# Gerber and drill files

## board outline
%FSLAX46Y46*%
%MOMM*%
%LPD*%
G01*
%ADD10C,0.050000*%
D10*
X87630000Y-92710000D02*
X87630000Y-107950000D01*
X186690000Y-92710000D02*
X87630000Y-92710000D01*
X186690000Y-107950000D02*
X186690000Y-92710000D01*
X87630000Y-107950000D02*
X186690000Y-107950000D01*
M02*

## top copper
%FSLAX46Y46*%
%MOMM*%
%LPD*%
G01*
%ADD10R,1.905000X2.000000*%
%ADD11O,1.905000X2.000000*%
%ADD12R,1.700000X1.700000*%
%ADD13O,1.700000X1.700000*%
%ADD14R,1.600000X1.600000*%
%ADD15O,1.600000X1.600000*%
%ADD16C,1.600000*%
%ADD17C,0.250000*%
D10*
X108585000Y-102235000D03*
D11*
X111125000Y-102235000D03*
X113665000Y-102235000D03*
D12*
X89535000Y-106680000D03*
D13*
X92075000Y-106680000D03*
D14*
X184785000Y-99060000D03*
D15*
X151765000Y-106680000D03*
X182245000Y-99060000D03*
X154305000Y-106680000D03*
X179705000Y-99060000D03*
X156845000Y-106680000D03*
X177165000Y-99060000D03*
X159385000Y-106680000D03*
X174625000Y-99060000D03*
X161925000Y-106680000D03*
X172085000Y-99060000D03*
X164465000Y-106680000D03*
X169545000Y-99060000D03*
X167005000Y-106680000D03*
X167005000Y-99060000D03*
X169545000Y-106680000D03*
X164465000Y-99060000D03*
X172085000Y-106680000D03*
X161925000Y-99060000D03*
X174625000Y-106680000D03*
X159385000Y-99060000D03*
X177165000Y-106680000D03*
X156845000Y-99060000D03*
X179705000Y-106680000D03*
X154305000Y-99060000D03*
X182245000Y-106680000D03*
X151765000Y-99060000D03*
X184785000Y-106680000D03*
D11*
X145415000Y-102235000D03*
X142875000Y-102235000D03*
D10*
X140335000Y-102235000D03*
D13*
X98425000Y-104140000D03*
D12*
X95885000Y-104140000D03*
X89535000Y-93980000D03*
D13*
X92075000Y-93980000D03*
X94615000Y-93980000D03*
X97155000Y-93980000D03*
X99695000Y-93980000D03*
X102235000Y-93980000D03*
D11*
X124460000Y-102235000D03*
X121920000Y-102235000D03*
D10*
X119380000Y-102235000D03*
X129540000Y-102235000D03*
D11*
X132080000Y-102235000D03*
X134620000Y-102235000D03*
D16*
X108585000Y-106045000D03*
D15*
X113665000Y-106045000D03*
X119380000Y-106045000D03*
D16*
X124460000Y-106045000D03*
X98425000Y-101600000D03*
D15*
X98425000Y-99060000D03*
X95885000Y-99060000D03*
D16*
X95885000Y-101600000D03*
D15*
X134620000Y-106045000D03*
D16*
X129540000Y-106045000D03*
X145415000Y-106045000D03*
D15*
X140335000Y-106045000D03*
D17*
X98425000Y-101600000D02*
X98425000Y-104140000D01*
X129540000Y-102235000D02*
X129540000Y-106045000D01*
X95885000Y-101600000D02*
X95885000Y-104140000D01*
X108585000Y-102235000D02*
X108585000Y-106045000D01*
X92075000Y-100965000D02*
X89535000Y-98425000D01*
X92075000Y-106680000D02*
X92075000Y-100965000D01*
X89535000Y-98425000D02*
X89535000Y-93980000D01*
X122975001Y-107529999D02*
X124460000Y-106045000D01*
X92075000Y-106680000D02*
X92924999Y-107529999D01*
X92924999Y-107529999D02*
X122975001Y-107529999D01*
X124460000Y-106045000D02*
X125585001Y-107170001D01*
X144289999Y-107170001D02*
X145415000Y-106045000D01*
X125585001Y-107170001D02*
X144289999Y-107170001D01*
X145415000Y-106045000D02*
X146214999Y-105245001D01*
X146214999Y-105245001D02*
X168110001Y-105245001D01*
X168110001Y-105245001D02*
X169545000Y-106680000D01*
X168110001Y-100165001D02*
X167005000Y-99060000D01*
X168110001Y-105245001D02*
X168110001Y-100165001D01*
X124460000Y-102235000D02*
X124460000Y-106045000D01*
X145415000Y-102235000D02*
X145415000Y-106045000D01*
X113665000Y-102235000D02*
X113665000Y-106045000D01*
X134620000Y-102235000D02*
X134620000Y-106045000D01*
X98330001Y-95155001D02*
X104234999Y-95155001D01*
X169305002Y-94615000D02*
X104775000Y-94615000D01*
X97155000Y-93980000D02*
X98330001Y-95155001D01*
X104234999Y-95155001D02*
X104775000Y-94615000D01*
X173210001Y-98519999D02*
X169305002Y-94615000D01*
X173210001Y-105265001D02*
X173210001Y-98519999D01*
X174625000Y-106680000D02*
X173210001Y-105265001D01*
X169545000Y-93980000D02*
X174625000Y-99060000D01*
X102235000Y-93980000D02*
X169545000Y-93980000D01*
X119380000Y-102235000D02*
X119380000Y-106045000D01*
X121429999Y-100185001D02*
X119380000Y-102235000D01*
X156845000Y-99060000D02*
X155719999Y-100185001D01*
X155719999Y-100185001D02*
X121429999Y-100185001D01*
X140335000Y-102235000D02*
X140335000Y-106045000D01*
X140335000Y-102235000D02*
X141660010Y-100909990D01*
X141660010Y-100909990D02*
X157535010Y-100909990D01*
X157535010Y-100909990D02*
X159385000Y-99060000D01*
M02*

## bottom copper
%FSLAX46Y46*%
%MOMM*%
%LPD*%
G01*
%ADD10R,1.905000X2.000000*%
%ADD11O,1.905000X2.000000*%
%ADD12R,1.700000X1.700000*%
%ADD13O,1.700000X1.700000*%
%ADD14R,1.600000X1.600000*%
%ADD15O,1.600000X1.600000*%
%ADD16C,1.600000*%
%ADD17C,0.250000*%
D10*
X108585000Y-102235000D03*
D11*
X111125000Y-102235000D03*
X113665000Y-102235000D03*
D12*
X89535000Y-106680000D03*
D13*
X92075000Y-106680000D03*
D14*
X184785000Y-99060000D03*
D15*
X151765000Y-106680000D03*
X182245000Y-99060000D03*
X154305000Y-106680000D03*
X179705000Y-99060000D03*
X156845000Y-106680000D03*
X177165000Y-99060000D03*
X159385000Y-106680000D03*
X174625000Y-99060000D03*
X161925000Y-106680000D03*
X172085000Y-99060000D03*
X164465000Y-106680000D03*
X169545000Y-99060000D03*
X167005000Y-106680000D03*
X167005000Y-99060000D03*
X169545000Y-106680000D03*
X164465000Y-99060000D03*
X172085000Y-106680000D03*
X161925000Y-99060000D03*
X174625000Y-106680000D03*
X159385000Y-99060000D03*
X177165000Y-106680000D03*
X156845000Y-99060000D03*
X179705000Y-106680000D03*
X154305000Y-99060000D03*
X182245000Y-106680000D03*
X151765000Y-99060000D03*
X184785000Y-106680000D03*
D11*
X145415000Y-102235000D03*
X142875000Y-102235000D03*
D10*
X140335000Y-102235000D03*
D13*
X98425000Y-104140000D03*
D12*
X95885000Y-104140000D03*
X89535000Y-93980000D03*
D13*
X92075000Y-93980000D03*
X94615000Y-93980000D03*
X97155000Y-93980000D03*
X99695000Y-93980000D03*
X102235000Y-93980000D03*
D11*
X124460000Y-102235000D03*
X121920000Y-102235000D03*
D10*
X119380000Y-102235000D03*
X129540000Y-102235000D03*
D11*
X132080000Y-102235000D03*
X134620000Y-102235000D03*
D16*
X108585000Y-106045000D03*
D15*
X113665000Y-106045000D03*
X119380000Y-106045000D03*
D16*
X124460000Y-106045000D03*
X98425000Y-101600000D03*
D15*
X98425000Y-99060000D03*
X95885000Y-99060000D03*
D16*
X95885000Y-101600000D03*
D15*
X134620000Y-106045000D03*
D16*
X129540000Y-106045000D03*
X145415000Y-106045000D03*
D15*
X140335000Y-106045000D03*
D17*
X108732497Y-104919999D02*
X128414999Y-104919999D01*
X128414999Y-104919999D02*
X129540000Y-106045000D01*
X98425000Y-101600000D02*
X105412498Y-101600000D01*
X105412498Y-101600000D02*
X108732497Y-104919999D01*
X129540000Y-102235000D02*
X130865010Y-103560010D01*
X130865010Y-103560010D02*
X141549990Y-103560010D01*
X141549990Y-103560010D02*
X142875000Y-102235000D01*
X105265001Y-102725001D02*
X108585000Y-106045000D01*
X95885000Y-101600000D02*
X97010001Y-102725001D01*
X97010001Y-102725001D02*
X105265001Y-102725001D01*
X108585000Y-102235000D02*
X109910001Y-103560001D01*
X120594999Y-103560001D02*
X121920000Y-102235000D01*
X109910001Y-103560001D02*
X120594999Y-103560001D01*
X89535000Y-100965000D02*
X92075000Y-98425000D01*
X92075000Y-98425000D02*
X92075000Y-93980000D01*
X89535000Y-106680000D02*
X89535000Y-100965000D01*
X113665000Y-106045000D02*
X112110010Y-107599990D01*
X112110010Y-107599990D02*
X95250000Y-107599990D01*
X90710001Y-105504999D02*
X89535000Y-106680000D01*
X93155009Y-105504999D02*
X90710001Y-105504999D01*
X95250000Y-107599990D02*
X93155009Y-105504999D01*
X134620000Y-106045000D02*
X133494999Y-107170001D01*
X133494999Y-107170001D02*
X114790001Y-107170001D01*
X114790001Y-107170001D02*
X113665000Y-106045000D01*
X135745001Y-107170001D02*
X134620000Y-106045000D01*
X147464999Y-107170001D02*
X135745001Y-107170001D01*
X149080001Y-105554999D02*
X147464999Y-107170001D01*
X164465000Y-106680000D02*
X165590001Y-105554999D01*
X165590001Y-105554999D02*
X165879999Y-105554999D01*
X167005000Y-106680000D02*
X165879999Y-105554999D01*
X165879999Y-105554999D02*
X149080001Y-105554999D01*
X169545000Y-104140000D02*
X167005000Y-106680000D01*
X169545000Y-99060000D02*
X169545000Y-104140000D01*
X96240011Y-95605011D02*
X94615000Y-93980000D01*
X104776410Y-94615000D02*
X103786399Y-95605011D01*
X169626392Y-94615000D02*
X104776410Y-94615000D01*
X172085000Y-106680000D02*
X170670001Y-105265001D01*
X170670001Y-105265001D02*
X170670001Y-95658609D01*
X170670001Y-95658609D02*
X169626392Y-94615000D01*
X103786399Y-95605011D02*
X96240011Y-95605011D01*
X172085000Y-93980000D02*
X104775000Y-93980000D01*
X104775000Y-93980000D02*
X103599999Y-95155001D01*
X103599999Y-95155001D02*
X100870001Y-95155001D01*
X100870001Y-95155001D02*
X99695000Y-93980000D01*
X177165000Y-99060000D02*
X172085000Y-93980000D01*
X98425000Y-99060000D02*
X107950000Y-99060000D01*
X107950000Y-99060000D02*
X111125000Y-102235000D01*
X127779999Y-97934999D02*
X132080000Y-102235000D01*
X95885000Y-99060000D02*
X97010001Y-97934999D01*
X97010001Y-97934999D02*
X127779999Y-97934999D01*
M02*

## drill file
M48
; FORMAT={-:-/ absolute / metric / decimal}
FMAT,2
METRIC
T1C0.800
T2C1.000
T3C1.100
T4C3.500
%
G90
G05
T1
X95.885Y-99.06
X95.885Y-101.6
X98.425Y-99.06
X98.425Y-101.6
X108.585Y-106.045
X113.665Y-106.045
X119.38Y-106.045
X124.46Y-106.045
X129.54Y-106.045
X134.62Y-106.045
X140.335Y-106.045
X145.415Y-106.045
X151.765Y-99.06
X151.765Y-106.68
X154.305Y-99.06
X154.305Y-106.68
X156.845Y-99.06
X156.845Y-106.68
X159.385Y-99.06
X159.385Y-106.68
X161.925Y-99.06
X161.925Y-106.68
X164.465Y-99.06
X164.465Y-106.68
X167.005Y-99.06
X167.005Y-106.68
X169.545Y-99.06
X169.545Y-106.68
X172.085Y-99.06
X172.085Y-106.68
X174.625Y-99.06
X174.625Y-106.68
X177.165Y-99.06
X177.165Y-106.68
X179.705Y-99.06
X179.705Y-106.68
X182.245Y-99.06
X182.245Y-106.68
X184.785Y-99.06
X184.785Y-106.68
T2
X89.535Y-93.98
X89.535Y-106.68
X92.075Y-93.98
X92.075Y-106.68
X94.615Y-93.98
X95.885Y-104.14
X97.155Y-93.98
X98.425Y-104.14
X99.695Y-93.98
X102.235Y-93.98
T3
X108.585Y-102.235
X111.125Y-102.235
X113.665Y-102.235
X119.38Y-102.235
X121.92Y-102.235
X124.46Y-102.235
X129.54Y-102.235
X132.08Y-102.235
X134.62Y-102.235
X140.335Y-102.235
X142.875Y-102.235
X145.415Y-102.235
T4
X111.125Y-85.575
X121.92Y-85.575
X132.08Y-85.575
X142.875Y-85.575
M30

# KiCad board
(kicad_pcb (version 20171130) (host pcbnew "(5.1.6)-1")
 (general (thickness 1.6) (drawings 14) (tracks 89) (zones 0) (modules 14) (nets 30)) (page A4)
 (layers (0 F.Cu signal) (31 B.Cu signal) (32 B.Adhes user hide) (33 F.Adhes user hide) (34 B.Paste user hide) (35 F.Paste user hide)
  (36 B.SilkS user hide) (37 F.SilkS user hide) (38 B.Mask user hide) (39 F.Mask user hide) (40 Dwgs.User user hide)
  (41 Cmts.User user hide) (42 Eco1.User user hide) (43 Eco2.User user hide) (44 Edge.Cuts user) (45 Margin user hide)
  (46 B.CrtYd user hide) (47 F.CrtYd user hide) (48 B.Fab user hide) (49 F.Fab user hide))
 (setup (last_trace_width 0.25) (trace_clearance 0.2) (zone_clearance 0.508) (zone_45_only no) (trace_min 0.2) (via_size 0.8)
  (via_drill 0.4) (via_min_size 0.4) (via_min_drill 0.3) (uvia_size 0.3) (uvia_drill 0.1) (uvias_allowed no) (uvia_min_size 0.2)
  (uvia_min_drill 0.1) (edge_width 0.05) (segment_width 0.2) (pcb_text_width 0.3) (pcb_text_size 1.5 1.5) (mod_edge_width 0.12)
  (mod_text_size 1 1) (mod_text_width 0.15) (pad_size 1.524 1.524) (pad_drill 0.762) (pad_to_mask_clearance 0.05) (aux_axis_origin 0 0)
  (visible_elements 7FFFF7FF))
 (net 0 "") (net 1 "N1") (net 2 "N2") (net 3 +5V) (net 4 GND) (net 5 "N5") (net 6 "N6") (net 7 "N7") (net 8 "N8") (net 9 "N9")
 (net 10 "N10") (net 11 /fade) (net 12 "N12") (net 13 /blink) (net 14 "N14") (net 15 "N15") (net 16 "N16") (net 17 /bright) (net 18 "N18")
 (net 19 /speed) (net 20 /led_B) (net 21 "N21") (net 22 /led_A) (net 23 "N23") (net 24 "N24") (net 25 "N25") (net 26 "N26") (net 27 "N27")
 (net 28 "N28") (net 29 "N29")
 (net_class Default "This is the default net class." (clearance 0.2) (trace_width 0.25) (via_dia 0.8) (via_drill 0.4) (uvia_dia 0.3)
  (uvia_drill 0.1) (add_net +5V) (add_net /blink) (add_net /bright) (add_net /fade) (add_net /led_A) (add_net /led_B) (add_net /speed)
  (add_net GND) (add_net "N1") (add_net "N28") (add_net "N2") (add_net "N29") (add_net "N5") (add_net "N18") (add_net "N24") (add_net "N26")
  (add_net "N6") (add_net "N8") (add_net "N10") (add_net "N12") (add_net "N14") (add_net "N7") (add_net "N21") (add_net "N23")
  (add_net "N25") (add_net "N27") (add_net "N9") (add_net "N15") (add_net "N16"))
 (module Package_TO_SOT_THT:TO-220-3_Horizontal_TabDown (layer F.Cu) (at 108.585 102.235)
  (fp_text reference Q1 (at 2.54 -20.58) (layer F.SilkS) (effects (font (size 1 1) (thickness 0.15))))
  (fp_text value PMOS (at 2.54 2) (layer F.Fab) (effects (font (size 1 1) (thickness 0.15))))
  (pad "" np_thru_hole oval (at 2.54 -16.66) (size 3.5 3.5) (drill 3.5) (layers *.Cu *.Mask))
  (pad 1 thru_hole rect (at 0 0) (size 1.905 2) (drill 1.1) (layers *.Cu *.Mask) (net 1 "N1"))
  (pad 2 thru_hole oval (at 2.54 0) (size 1.905 2) (drill 1.1) (layers *.Cu *.Mask) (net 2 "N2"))
  (pad 3 thru_hole oval (at 5.08 0) (size 1.905 2) (drill 1.1) (layers *.Cu *.Mask) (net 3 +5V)))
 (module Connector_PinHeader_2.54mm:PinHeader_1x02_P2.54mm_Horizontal (layer F.Cu) (at 89.535 106.68 90)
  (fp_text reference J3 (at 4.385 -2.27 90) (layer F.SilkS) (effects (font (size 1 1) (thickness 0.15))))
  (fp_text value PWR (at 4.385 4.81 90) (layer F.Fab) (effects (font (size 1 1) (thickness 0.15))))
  (pad 1 thru_hole rect (at 0 0 90) (size 1.7 1.7) (drill 1) (layers *.Cu *.Mask) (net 3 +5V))
  (pad 2 thru_hole oval (at 0 2.54 90) (size 1.7 1.7) (drill 1) (layers *.Cu *.Mask) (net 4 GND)))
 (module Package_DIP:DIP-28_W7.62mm (layer F.Cu) (at 184.785 99.06 270)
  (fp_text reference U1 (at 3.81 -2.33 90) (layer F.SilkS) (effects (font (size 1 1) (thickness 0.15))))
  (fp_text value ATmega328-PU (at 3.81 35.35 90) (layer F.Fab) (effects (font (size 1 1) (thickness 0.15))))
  (pad 1 thru_hole rect (at 0 0 270) (size 1.6 1.6) (drill 0.8) (layers *.Cu *.Mask) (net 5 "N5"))
  (pad 15 thru_hole oval (at 7.62 33.02 270) (size 1.6 1.6) (drill 0.8) (layers *.Cu *.Mask) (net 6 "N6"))
  (pad 2 thru_hole oval (at 0 2.54 270) (size 1.6 1.6) (drill 0.8) (layers *.Cu *.Mask) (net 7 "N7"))
  (pad 16 thru_hole oval (at 7.62 30.48 270) (size 1.6 1.6) (drill 0.8) (layers *.Cu *.Mask) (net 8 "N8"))
  (pad 3 thru_hole oval (at 0 5.08 270) (size 1.6 1.6) (drill 0.8) (layers *.Cu *.Mask) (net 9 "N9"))
  (pad 17 thru_hole oval (at 7.62 27.94 270) (size 1.6 1.6) (drill 0.8) (layers *.Cu *.Mask) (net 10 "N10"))
  (pad 4 thru_hole oval (at 0 7.62 270) (size 1.6 1.6) (drill 0.8) (layers *.Cu *.Mask) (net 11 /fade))
  (pad 18 thru_hole oval (at 7.62 25.4 270) (size 1.6 1.6) (drill 0.8) (layers *.Cu *.Mask) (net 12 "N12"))
  (pad 5 thru_hole oval (at 0 10.16 270) (size 1.6 1.6) (drill 0.8) (layers *.Cu *.Mask) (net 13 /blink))
  (pad 19 thru_hole oval (at 7.62 22.86 270) (size 1.6 1.6) (drill 0.8) (layers *.Cu *.Mask) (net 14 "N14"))
  (pad 6 thru_hole oval (at 0 12.7 270) (size 1.6 1.6) (drill 0.8) (layers *.Cu *.Mask) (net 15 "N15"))
  (pad 20 thru_hole oval (at 7.62 20.32 270) (size 1.6 1.6) (drill 0.8) (layers *.Cu *.Mask) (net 3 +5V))
  (pad 7 thru_hole oval (at 0 15.24 270) (size 1.6 1.6) (drill 0.8) (layers *.Cu *.Mask) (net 3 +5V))
  (pad 21 thru_hole oval (at 7.62 17.78 270) (size 1.6 1.6) (drill 0.8) (layers *.Cu *.Mask) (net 3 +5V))
  (pad 8 thru_hole oval (at 0 17.78 270) (size 1.6 1.6) (drill 0.8) (layers *.Cu *.Mask) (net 4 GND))
  (pad 22 thru_hole oval (at 7.62 15.24 270) (size 1.6 1.6) (drill 0.8) (layers *.Cu *.Mask) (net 4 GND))
  (pad 9 thru_hole oval (at 0 20.32 270) (size 1.6 1.6) (drill 0.8) (layers *.Cu *.Mask) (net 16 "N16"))
  (pad 23 thru_hole oval (at 7.62 12.7 270) (size 1.6 1.6) (drill 0.8) (layers *.Cu *.Mask) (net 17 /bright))
  (pad 10 thru_hole oval (at 0 22.86 270) (size 1.6 1.6) (drill 0.8) (layers *.Cu *.Mask) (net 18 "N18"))
  (pad 24 thru_hole oval (at 7.62 10.16 270) (size 1.6 1.6) (drill 0.8) (layers *.Cu *.Mask) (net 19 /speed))
  (pad 11 thru_hole oval (at 0 25.4 270) (size 1.6 1.6) (drill 0.8) (layers *.Cu *.Mask) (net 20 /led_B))
  (pad 25 thru_hole oval (at 7.62 7.62 270) (size 1.6 1.6) (drill 0.8) (layers *.Cu *.Mask) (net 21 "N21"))
  (pad 12 thru_hole oval (at 0 27.94 270) (size 1.6 1.6) (drill 0.8) (layers *.Cu *.Mask) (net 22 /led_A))
  (pad 26 thru_hole oval (at 7.62 5.08 270) (size 1.6 1.6) (drill 0.8) (layers *.Cu *.Mask) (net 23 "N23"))
  (pad 13 thru_hole oval (at 0 30.48 270) (size 1.6 1.6) (drill 0.8) (layers *.Cu *.Mask) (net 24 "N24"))
  (pad 27 thru_hole oval (at 7.62 2.54 270) (size 1.6 1.6) (drill 0.8) (layers *.Cu *.Mask) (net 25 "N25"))
  (pad 14 thru_hole oval (at 0 33.02 270) (size 1.6 1.6) (drill 0.8) (layers *.Cu *.Mask) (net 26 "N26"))
  (pad 28 thru_hole oval (at 7.62 0 270) (size 1.6 1.6) (drill 0.8) (layers *.Cu *.Mask) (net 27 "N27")))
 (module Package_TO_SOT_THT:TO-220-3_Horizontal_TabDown (layer F.Cu) (at 140.335 102.235)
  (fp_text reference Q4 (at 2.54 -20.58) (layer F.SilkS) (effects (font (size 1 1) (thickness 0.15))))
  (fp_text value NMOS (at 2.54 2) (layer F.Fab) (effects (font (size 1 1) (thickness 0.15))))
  (pad 3 thru_hole oval (at 5.08 0) (size 1.905 2) (drill 1.1) (layers *.Cu *.Mask) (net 4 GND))
  (pad 2 thru_hole oval (at 2.54 0) (size 1.905 2) (drill 1.1) (layers *.Cu *.Mask) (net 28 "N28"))
  (pad 1 thru_hole rect (at 0 0) (size 1.905 2) (drill 1.1) (layers *.Cu *.Mask) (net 20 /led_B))
  (pad "" np_thru_hole oval (at 2.54 -16.66) (size 3.5 3.5) (drill 3.5) (layers *.Cu *.Mask)))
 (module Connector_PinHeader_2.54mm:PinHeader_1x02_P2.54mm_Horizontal (layer F.Cu) (at 95.885 104.14 90)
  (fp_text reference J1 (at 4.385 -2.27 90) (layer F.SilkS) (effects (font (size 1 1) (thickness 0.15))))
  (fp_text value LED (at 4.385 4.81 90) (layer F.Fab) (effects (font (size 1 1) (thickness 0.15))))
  (pad 2 thru_hole oval (at 0 2.54 90) (size 1.7 1.7) (drill 1) (layers *.Cu *.Mask) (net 28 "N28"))
  (pad 1 thru_hole rect (at 0 0 90) (size 1.7 1.7) (drill 1) (layers *.Cu *.Mask) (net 1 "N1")))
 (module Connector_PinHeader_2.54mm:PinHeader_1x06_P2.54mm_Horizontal (layer F.Cu) (at 89.535 93.98 90)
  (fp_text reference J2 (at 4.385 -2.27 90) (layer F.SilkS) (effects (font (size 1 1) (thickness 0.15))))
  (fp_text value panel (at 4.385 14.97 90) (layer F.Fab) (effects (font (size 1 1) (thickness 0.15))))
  (pad 1 thru_hole rect (at 0 0 90) (size 1.7 1.7) (drill 1) (layers *.Cu *.Mask) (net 4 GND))
  (pad 2 thru_hole oval (at 0 2.54 90) (size 1.7 1.7) (drill 1) (layers *.Cu *.Mask) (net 3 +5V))
  (pad 3 thru_hole oval (at 0 5.08 90) (size 1.7 1.7) (drill 1) (layers *.Cu *.Mask) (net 17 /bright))
  (pad 4 thru_hole oval (at 0 7.62 90) (size 1.7 1.7) (drill 1) (layers *.Cu *.Mask) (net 19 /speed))
  (pad 5 thru_hole oval (at 0 10.16 90) (size 1.7 1.7) (drill 1) (layers *.Cu *.Mask) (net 11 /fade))
  (pad 6 thru_hole oval (at 0 12.7 90) (size 1.7 1.7) (drill 1) (layers *.Cu *.Mask) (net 13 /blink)))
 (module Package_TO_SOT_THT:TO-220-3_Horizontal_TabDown (layer F.Cu) (at 119.38 102.235)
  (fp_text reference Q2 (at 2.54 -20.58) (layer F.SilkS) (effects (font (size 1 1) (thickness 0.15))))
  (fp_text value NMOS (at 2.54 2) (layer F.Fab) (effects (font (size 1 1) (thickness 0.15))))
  (pad 3 thru_hole oval (at 5.08 0) (size 1.905 2) (drill 1.1) (layers *.Cu *.Mask) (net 4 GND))
  (pad 2 thru_hole oval (at 2.54 0) (size 1.905 2) (drill 1.1) (layers *.Cu *.Mask) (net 1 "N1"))
  (pad 1 thru_hole rect (at 0 0) (size 1.905 2) (drill 1.1) (layers *.Cu *.Mask) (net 22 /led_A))
  (pad "" np_thru_hole oval (at 2.54 -16.66) (size 3.5 3.5) (drill 3.5) (layers *.Cu *.Mask)))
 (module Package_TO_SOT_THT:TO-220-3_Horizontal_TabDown (layer F.Cu) (at 129.54 102.235)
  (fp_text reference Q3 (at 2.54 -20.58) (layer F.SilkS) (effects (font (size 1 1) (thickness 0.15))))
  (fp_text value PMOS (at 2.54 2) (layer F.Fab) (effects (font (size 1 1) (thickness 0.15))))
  (pad "" np_thru_hole oval (at 2.54 -16.66) (size 3.5 3.5) (drill 3.5) (layers *.Cu *.Mask))
  (pad 1 thru_hole rect (at 0 0) (size 1.905 2) (drill 1.1) (layers *.Cu *.Mask) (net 28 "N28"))
  (pad 2 thru_hole oval (at 2.54 0) (size 1.905 2) (drill 1.1) (layers *.Cu *.Mask) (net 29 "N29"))
  (pad 3 thru_hole oval (at 5.08 0) (size 1.905 2) (drill 1.1) (layers *.Cu *.Mask) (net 3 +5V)))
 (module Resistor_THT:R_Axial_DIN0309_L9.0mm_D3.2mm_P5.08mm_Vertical (layer F.Cu) (at 108.585 106.045)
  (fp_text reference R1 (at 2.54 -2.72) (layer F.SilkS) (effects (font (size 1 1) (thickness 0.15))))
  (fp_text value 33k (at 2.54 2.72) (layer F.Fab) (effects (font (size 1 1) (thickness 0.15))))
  (pad 1 thru_hole circle (at 0 0) (size 1.6 1.6) (drill 0.8) (layers *.Cu *.Mask) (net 1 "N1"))
  (pad 2 thru_hole oval (at 5.08 0) (size 1.6 1.6) (drill 0.8) (layers *.Cu *.Mask) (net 3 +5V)))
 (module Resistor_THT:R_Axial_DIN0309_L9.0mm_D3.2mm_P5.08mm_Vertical (layer F.Cu) (at 124.46 106.045 180)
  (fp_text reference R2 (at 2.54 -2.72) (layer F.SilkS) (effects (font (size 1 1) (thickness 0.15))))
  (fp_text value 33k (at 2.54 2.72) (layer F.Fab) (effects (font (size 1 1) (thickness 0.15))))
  (pad 2 thru_hole oval (at 5.08 0 180) (size 1.6 1.6) (drill 0.8) (layers *.Cu *.Mask) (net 22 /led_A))
  (pad 1 thru_hole circle (at 0 0 180) (size 1.6 1.6) (drill 0.8) (layers *.Cu *.Mask) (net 4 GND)))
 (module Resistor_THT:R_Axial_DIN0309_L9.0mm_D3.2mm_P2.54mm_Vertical (layer F.Cu) (at 98.425 101.6 90)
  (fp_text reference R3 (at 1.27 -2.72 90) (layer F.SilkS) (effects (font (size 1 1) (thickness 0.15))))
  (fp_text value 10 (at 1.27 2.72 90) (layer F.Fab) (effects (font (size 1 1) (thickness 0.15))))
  (pad 1 thru_hole circle (at 0 0 90) (size 1.6 1.6) (drill 0.8) (layers *.Cu *.Mask) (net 28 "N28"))
  (pad 2 thru_hole oval (at 2.54 0 90) (size 1.6 1.6) (drill 0.8) (layers *.Cu *.Mask) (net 2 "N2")))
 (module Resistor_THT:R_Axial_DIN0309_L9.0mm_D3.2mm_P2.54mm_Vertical (layer F.Cu) (at 95.885 101.6 90)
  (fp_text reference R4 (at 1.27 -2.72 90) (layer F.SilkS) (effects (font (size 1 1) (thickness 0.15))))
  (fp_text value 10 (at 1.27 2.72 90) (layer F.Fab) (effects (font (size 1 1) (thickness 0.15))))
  (pad 2 thru_hole oval (at 2.54 0 90) (size 1.6 1.6) (drill 0.8) (layers *.Cu *.Mask) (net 29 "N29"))
  (pad 1 thru_hole circle (at 0 0 90) (size 1.6 1.6) (drill 0.8) (layers *.Cu *.Mask) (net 1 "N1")))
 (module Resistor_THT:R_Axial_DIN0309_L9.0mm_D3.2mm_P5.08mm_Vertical (layer F.Cu) (at 129.54 106.045)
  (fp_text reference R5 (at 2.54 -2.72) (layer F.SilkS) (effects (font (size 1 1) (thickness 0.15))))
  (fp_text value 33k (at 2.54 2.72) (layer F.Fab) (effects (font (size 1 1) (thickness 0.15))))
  (pad 2 thru_hole oval (at 5.08 0) (size 1.6 1.6) (drill 0.8) (layers *.Cu *.Mask) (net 3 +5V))
  (pad 1 thru_hole circle (at 0 0) (size 1.6 1.6) (drill 0.8) (layers *.Cu *.Mask) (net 28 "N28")))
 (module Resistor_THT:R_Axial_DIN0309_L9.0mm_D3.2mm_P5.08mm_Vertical (layer F.Cu) (at 145.415 106.045 180)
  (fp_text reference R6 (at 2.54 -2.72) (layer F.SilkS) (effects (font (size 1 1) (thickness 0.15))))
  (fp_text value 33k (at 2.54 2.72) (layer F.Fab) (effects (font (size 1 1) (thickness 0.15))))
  (pad 1 thru_hole circle (at 0 0 180) (size 1.6 1.6) (drill 0.8) (layers *.Cu *.Mask) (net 4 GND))
  (pad 2 thru_hole oval (at 5.08 0 180) (size 1.6 1.6) (drill 0.8) (layers *.Cu *.Mask) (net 20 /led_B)))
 (gr_line (start 87.63 92.71) (end 87.63 107.95) (layer Edge.Cuts) (width 0.05))
 (gr_line (start 186.69 92.71) (end 87.63 92.71) (layer Edge.Cuts) (width 0.05))
 (gr_line (start 186.69 107.95) (end 186.69 92.71) (layer Edge.Cuts) (width 0.05))
 (gr_line (start 87.63 107.95) (end 186.69 107.95) (layer Edge.Cuts) (width 0.05))
 (segment (start 108.732497 104.919999) (end 128.414999 104.919999) (width 0.25) (layer B.Cu) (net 28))
 (segment (start 128.414999 104.919999) (end 129.54 106.045) (width 0.25) (layer B.Cu) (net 28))
 (segment (start 98.425 101.6) (end 105.412498 101.6) (width 0.25) (layer B.Cu) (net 28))
 (segment (start 105.412498 101.6) (end 108.732497 104.919999) (width 0.25) (layer B.Cu) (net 28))
 (segment (start 98.425 101.6) (end 98.425 104.14) (width 0.25) (layer F.Cu) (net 28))
 (segment (start 129.54 102.235) (end 129.54 106.045) (width 0.25) (layer F.Cu) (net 28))
 (segment (start 129.54 102.235) (end 130.86501 103.56001) (width 0.25) (layer B.Cu) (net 28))
 (segment (start 130.86501 103.56001) (end 141.54999 103.56001) (width 0.25) (layer B.Cu) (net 28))
 (segment (start 141.54999 103.56001) (end 142.875 102.235) (width 0.25) (layer B.Cu) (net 28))
 (segment (start 105.265001 102.725001) (end 108.585 106.045) (width 0.25) (layer B.Cu) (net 1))
 (segment (start 95.885 101.6) (end 97.010001 102.725001) (width 0.25) (layer B.Cu) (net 1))
 (segment (start 95.885 101.6) (end 95.885 104.14) (width 0.25) (layer F.Cu) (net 1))
 (segment (start 97.010001 102.725001) (end 105.265001 102.725001) (width 0.25) (layer B.Cu) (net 1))
 (segment (start 108.585 102.235) (end 108.585 106.045) (width 0.25) (layer F.Cu) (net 1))
 (segment (start 108.585 102.235) (end 109.910001 103.560001) (width 0.25) (layer B.Cu) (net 1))
 (segment (start 120.594999 103.560001) (end 121.92 102.235) (width 0.25) (layer B.Cu) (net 1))
 (segment (start 109.910001 103.560001) (end 120.594999 103.560001) (width 0.25) (layer B.Cu) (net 1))
 (segment (start 92.075 100.965) (end 89.535 98.425) (width 0.25) (layer F.Cu) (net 4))
 (segment (start 92.075 106.68) (end 92.075 100.965) (width 0.25) (layer F.Cu) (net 4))
 (segment (start 89.535 98.425) (end 89.535 93.98) (width 0.25) (layer F.Cu) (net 4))
 (segment (start 122.975001 107.529999) (end 124.46 106.045) (width 0.25) (layer F.Cu) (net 4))
 (segment (start 92.075 106.68) (end 92.924999 107.529999) (width 0.25) (layer F.Cu) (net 4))
 (segment (start 92.924999 107.529999) (end 122.975001 107.529999) (width 0.25) (layer F.Cu) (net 4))
 (segment (start 124.46 106.045) (end 125.585001 107.170001) (width 0.25) (layer F.Cu) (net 4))
 (segment (start 144.289999 107.170001) (end 145.415 106.045) (width 0.25) (layer F.Cu) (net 4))
 (segment (start 125.585001 107.170001) (end 144.289999 107.170001) (width 0.25) (layer F.Cu) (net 4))
 (segment (start 145.415 106.045) (end 146.214999 105.245001) (width 0.25) (layer F.Cu) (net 4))
 (segment (start 146.214999 105.245001) (end 168.110001 105.245001) (width 0.25) (layer F.Cu) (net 4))
 (segment (start 168.110001 105.245001) (end 169.545 106.68) (width 0.25) (layer F.Cu) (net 4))
 (segment (start 168.110001 100.165001) (end 167.005 99.06) (width 0.25) (layer F.Cu) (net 4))
 (segment (start 168.110001 105.245001) (end 168.110001 100.165001) (width 0.25) (layer F.Cu) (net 4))
 (segment (start 124.46 102.235) (end 124.46 106.045) (width 0.25) (layer F.Cu) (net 4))
 (segment (start 145.415 102.235) (end 145.415 106.045) (width 0.25) (layer F.Cu) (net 4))
 (segment (start 89.535 100.965) (end 92.075 98.425) (width 0.25) (layer B.Cu) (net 3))
 (segment (start 92.075 98.425) (end 92.075 93.98) (width 0.25) (layer B.Cu) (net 3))
 (segment (start 89.535 106.68) (end 89.535 100.965) (width 0.25) (layer B.Cu) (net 3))
 (segment (start 113.665 106.045) (end 112.11001 107.59999) (width 0.25) (layer B.Cu) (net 3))
 (segment (start 112.11001 107.59999) (end 95.25 107.59999) (width 0.25) (layer B.Cu) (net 3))
 (segment (start 90.710001 105.504999) (end 89.535 106.68) (width 0.25) (layer B.Cu) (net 3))
 (segment (start 93.155009 105.504999) (end 90.710001 105.504999) (width 0.25) (layer B.Cu) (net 3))
 (segment (start 95.25 107.59999) (end 93.155009 105.504999) (width 0.25) (layer B.Cu) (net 3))
 (segment (start 134.62 106.045) (end 133.494999 107.170001) (width 0.25) (layer B.Cu) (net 3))
 (segment (start 133.494999 107.170001) (end 114.790001 107.170001) (width 0.25) (layer B.Cu) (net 3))
 (segment (start 114.790001 107.170001) (end 113.665 106.045) (width 0.25) (layer B.Cu) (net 3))
 (segment (start 135.745001 107.170001) (end 134.62 106.045) (width 0.25) (layer B.Cu) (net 3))
 (segment (start 147.464999 107.170001) (end 135.745001 107.170001) (width 0.25) (layer B.Cu) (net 3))
 (segment (start 149.080001 105.554999) (end 147.464999 107.170001) (width 0.25) (layer B.Cu) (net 3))
 (segment (start 164.465 106.68) (end 165.590001 105.554999) (width 0.25) (layer B.Cu) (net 3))
 (segment (start 165.590001 105.554999) (end 165.879999 105.554999) (width 0.25) (layer B.Cu) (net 3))
 (segment (start 167.005 106.68) (end 165.879999 105.554999) (width 0.25) (layer B.Cu) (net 3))
 (segment (start 165.879999 105.554999) (end 149.080001 105.554999) (width 0.25) (layer B.Cu) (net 3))
 (segment (start 169.545 104.14) (end 167.005 106.68) (width 0.25) (layer B.Cu) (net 3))
 (segment (start 169.545 99.06) (end 169.545 104.14) (width 0.25) (layer B.Cu) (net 3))
 (segment (start 113.665 102.235) (end 113.665 106.045) (width 0.25) (layer F.Cu) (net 3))
 (segment (start 134.62 102.235) (end 134.62 106.045) (width 0.25) (layer F.Cu) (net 3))
 (segment (start 96.240011 95.605011) (end 94.615 93.98) (width 0.25) (layer B.Cu) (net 17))
 (segment (start 104.77641 94.615) (end 103.786399 95.605011) (width 0.25) (layer B.Cu) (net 17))
 (segment (start 169.626392 94.615) (end 104.77641 94.615) (width 0.25) (layer B.Cu) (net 17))
 (segment (start 172.085 106.68) (end 170.670001 105.265001) (width 0.25) (layer B.Cu) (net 17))
 (segment (start 170.670001 105.265001) (end 170.670001 95.658609) (width 0.25) (layer B.Cu) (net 17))
 (segment (start 170.670001 95.658609) (end 169.626392 94.615) (width 0.25) (layer B.Cu) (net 17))
 (segment (start 103.786399 95.605011) (end 96.240011 95.605011) (width 0.25) (layer B.Cu) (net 17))
 (segment (start 98.330001 95.155001) (end 104.234999 95.155001) (width 0.25) (layer F.Cu) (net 19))
 (segment (start 169.305002 94.615) (end 104.775 94.615) (width 0.25) (layer F.Cu) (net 19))
 (segment (start 97.155 93.98) (end 98.330001 95.155001) (width 0.25) (layer F.Cu) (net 19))
 (segment (start 104.234999 95.155001) (end 104.775 94.615) (width 0.25) (layer F.Cu) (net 19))
 (segment (start 173.210001 98.519999) (end 169.305002 94.615) (width 0.25) (layer F.Cu) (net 19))
 (segment (start 173.210001 105.265001) (end 173.210001 98.519999) (width 0.25) (layer F.Cu) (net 19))
 (segment (start 174.625 106.68) (end 173.210001 105.265001) (width 0.25) (layer F.Cu) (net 19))
 (segment (start 172.085 93.98) (end 104.775 93.98) (width 0.25) (layer B.Cu) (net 11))
 (segment (start 104.775 93.98) (end 103.599999 95.155001) (width 0.25) (layer B.Cu) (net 11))
 (segment (start 103.599999 95.155001) (end 100.870001 95.155001) (width 0.25) (layer B.Cu) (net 11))
 (segment (start 100.870001 95.155001) (end 99.695 93.98) (width 0.25) (layer B.Cu) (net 11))
 (segment (start 177.165 99.06) (end 172.085 93.98) (width 0.25) (layer B.Cu) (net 11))
 (segment (start 169.545 93.98) (end 174.625 99.06) (width 0.25) (layer F.Cu) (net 13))
 (segment (start 102.235 93.98) (end 169.545 93.98) (width 0.25) (layer F.Cu) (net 13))
 (segment (start 98.425 99.06) (end 107.95 99.06) (width 0.25) (layer B.Cu) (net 2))
 (segment (start 107.95 99.06) (end 111.125 102.235) (width 0.25) (layer B.Cu) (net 2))
 (segment (start 119.38 102.235) (end 119.38 106.045) (width 0.25) (layer F.Cu) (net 22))
 (segment (start 121.429999 100.185001) (end 119.38 102.235) (width 0.25) (layer F.Cu) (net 22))
 (segment (start 156.845 99.06) (end 155.719999 100.185001) (width 0.25) (layer F.Cu) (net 22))
 (segment (start 155.719999 100.185001) (end 121.429999 100.185001) (width 0.25) (layer F.Cu) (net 22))
 (segment (start 127.779999 97.934999) (end 132.08 102.235) (width 0.25) (layer B.Cu) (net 29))
 (segment (start 95.885 99.06) (end 97.010001 97.934999) (width 0.25) (layer B.Cu) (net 29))
 (segment (start 97.010001 97.934999) (end 127.779999 97.934999) (width 0.25) (layer B.Cu) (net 29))
 (segment (start 140.335 102.235) (end 140.335 106.045) (width 0.25) (layer F.Cu) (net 20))
 (segment (start 140.335 102.235) (end 141.66001 100.90999) (width 0.25) (layer F.Cu) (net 20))
 (segment (start 141.66001 100.90999) (end 157.53501 100.90999) (width 0.25) (layer F.Cu) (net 20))
 (segment (start 157.53501 100.90999) (end 159.385 99.06) (width 0.25) (layer F.Cu) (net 20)))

